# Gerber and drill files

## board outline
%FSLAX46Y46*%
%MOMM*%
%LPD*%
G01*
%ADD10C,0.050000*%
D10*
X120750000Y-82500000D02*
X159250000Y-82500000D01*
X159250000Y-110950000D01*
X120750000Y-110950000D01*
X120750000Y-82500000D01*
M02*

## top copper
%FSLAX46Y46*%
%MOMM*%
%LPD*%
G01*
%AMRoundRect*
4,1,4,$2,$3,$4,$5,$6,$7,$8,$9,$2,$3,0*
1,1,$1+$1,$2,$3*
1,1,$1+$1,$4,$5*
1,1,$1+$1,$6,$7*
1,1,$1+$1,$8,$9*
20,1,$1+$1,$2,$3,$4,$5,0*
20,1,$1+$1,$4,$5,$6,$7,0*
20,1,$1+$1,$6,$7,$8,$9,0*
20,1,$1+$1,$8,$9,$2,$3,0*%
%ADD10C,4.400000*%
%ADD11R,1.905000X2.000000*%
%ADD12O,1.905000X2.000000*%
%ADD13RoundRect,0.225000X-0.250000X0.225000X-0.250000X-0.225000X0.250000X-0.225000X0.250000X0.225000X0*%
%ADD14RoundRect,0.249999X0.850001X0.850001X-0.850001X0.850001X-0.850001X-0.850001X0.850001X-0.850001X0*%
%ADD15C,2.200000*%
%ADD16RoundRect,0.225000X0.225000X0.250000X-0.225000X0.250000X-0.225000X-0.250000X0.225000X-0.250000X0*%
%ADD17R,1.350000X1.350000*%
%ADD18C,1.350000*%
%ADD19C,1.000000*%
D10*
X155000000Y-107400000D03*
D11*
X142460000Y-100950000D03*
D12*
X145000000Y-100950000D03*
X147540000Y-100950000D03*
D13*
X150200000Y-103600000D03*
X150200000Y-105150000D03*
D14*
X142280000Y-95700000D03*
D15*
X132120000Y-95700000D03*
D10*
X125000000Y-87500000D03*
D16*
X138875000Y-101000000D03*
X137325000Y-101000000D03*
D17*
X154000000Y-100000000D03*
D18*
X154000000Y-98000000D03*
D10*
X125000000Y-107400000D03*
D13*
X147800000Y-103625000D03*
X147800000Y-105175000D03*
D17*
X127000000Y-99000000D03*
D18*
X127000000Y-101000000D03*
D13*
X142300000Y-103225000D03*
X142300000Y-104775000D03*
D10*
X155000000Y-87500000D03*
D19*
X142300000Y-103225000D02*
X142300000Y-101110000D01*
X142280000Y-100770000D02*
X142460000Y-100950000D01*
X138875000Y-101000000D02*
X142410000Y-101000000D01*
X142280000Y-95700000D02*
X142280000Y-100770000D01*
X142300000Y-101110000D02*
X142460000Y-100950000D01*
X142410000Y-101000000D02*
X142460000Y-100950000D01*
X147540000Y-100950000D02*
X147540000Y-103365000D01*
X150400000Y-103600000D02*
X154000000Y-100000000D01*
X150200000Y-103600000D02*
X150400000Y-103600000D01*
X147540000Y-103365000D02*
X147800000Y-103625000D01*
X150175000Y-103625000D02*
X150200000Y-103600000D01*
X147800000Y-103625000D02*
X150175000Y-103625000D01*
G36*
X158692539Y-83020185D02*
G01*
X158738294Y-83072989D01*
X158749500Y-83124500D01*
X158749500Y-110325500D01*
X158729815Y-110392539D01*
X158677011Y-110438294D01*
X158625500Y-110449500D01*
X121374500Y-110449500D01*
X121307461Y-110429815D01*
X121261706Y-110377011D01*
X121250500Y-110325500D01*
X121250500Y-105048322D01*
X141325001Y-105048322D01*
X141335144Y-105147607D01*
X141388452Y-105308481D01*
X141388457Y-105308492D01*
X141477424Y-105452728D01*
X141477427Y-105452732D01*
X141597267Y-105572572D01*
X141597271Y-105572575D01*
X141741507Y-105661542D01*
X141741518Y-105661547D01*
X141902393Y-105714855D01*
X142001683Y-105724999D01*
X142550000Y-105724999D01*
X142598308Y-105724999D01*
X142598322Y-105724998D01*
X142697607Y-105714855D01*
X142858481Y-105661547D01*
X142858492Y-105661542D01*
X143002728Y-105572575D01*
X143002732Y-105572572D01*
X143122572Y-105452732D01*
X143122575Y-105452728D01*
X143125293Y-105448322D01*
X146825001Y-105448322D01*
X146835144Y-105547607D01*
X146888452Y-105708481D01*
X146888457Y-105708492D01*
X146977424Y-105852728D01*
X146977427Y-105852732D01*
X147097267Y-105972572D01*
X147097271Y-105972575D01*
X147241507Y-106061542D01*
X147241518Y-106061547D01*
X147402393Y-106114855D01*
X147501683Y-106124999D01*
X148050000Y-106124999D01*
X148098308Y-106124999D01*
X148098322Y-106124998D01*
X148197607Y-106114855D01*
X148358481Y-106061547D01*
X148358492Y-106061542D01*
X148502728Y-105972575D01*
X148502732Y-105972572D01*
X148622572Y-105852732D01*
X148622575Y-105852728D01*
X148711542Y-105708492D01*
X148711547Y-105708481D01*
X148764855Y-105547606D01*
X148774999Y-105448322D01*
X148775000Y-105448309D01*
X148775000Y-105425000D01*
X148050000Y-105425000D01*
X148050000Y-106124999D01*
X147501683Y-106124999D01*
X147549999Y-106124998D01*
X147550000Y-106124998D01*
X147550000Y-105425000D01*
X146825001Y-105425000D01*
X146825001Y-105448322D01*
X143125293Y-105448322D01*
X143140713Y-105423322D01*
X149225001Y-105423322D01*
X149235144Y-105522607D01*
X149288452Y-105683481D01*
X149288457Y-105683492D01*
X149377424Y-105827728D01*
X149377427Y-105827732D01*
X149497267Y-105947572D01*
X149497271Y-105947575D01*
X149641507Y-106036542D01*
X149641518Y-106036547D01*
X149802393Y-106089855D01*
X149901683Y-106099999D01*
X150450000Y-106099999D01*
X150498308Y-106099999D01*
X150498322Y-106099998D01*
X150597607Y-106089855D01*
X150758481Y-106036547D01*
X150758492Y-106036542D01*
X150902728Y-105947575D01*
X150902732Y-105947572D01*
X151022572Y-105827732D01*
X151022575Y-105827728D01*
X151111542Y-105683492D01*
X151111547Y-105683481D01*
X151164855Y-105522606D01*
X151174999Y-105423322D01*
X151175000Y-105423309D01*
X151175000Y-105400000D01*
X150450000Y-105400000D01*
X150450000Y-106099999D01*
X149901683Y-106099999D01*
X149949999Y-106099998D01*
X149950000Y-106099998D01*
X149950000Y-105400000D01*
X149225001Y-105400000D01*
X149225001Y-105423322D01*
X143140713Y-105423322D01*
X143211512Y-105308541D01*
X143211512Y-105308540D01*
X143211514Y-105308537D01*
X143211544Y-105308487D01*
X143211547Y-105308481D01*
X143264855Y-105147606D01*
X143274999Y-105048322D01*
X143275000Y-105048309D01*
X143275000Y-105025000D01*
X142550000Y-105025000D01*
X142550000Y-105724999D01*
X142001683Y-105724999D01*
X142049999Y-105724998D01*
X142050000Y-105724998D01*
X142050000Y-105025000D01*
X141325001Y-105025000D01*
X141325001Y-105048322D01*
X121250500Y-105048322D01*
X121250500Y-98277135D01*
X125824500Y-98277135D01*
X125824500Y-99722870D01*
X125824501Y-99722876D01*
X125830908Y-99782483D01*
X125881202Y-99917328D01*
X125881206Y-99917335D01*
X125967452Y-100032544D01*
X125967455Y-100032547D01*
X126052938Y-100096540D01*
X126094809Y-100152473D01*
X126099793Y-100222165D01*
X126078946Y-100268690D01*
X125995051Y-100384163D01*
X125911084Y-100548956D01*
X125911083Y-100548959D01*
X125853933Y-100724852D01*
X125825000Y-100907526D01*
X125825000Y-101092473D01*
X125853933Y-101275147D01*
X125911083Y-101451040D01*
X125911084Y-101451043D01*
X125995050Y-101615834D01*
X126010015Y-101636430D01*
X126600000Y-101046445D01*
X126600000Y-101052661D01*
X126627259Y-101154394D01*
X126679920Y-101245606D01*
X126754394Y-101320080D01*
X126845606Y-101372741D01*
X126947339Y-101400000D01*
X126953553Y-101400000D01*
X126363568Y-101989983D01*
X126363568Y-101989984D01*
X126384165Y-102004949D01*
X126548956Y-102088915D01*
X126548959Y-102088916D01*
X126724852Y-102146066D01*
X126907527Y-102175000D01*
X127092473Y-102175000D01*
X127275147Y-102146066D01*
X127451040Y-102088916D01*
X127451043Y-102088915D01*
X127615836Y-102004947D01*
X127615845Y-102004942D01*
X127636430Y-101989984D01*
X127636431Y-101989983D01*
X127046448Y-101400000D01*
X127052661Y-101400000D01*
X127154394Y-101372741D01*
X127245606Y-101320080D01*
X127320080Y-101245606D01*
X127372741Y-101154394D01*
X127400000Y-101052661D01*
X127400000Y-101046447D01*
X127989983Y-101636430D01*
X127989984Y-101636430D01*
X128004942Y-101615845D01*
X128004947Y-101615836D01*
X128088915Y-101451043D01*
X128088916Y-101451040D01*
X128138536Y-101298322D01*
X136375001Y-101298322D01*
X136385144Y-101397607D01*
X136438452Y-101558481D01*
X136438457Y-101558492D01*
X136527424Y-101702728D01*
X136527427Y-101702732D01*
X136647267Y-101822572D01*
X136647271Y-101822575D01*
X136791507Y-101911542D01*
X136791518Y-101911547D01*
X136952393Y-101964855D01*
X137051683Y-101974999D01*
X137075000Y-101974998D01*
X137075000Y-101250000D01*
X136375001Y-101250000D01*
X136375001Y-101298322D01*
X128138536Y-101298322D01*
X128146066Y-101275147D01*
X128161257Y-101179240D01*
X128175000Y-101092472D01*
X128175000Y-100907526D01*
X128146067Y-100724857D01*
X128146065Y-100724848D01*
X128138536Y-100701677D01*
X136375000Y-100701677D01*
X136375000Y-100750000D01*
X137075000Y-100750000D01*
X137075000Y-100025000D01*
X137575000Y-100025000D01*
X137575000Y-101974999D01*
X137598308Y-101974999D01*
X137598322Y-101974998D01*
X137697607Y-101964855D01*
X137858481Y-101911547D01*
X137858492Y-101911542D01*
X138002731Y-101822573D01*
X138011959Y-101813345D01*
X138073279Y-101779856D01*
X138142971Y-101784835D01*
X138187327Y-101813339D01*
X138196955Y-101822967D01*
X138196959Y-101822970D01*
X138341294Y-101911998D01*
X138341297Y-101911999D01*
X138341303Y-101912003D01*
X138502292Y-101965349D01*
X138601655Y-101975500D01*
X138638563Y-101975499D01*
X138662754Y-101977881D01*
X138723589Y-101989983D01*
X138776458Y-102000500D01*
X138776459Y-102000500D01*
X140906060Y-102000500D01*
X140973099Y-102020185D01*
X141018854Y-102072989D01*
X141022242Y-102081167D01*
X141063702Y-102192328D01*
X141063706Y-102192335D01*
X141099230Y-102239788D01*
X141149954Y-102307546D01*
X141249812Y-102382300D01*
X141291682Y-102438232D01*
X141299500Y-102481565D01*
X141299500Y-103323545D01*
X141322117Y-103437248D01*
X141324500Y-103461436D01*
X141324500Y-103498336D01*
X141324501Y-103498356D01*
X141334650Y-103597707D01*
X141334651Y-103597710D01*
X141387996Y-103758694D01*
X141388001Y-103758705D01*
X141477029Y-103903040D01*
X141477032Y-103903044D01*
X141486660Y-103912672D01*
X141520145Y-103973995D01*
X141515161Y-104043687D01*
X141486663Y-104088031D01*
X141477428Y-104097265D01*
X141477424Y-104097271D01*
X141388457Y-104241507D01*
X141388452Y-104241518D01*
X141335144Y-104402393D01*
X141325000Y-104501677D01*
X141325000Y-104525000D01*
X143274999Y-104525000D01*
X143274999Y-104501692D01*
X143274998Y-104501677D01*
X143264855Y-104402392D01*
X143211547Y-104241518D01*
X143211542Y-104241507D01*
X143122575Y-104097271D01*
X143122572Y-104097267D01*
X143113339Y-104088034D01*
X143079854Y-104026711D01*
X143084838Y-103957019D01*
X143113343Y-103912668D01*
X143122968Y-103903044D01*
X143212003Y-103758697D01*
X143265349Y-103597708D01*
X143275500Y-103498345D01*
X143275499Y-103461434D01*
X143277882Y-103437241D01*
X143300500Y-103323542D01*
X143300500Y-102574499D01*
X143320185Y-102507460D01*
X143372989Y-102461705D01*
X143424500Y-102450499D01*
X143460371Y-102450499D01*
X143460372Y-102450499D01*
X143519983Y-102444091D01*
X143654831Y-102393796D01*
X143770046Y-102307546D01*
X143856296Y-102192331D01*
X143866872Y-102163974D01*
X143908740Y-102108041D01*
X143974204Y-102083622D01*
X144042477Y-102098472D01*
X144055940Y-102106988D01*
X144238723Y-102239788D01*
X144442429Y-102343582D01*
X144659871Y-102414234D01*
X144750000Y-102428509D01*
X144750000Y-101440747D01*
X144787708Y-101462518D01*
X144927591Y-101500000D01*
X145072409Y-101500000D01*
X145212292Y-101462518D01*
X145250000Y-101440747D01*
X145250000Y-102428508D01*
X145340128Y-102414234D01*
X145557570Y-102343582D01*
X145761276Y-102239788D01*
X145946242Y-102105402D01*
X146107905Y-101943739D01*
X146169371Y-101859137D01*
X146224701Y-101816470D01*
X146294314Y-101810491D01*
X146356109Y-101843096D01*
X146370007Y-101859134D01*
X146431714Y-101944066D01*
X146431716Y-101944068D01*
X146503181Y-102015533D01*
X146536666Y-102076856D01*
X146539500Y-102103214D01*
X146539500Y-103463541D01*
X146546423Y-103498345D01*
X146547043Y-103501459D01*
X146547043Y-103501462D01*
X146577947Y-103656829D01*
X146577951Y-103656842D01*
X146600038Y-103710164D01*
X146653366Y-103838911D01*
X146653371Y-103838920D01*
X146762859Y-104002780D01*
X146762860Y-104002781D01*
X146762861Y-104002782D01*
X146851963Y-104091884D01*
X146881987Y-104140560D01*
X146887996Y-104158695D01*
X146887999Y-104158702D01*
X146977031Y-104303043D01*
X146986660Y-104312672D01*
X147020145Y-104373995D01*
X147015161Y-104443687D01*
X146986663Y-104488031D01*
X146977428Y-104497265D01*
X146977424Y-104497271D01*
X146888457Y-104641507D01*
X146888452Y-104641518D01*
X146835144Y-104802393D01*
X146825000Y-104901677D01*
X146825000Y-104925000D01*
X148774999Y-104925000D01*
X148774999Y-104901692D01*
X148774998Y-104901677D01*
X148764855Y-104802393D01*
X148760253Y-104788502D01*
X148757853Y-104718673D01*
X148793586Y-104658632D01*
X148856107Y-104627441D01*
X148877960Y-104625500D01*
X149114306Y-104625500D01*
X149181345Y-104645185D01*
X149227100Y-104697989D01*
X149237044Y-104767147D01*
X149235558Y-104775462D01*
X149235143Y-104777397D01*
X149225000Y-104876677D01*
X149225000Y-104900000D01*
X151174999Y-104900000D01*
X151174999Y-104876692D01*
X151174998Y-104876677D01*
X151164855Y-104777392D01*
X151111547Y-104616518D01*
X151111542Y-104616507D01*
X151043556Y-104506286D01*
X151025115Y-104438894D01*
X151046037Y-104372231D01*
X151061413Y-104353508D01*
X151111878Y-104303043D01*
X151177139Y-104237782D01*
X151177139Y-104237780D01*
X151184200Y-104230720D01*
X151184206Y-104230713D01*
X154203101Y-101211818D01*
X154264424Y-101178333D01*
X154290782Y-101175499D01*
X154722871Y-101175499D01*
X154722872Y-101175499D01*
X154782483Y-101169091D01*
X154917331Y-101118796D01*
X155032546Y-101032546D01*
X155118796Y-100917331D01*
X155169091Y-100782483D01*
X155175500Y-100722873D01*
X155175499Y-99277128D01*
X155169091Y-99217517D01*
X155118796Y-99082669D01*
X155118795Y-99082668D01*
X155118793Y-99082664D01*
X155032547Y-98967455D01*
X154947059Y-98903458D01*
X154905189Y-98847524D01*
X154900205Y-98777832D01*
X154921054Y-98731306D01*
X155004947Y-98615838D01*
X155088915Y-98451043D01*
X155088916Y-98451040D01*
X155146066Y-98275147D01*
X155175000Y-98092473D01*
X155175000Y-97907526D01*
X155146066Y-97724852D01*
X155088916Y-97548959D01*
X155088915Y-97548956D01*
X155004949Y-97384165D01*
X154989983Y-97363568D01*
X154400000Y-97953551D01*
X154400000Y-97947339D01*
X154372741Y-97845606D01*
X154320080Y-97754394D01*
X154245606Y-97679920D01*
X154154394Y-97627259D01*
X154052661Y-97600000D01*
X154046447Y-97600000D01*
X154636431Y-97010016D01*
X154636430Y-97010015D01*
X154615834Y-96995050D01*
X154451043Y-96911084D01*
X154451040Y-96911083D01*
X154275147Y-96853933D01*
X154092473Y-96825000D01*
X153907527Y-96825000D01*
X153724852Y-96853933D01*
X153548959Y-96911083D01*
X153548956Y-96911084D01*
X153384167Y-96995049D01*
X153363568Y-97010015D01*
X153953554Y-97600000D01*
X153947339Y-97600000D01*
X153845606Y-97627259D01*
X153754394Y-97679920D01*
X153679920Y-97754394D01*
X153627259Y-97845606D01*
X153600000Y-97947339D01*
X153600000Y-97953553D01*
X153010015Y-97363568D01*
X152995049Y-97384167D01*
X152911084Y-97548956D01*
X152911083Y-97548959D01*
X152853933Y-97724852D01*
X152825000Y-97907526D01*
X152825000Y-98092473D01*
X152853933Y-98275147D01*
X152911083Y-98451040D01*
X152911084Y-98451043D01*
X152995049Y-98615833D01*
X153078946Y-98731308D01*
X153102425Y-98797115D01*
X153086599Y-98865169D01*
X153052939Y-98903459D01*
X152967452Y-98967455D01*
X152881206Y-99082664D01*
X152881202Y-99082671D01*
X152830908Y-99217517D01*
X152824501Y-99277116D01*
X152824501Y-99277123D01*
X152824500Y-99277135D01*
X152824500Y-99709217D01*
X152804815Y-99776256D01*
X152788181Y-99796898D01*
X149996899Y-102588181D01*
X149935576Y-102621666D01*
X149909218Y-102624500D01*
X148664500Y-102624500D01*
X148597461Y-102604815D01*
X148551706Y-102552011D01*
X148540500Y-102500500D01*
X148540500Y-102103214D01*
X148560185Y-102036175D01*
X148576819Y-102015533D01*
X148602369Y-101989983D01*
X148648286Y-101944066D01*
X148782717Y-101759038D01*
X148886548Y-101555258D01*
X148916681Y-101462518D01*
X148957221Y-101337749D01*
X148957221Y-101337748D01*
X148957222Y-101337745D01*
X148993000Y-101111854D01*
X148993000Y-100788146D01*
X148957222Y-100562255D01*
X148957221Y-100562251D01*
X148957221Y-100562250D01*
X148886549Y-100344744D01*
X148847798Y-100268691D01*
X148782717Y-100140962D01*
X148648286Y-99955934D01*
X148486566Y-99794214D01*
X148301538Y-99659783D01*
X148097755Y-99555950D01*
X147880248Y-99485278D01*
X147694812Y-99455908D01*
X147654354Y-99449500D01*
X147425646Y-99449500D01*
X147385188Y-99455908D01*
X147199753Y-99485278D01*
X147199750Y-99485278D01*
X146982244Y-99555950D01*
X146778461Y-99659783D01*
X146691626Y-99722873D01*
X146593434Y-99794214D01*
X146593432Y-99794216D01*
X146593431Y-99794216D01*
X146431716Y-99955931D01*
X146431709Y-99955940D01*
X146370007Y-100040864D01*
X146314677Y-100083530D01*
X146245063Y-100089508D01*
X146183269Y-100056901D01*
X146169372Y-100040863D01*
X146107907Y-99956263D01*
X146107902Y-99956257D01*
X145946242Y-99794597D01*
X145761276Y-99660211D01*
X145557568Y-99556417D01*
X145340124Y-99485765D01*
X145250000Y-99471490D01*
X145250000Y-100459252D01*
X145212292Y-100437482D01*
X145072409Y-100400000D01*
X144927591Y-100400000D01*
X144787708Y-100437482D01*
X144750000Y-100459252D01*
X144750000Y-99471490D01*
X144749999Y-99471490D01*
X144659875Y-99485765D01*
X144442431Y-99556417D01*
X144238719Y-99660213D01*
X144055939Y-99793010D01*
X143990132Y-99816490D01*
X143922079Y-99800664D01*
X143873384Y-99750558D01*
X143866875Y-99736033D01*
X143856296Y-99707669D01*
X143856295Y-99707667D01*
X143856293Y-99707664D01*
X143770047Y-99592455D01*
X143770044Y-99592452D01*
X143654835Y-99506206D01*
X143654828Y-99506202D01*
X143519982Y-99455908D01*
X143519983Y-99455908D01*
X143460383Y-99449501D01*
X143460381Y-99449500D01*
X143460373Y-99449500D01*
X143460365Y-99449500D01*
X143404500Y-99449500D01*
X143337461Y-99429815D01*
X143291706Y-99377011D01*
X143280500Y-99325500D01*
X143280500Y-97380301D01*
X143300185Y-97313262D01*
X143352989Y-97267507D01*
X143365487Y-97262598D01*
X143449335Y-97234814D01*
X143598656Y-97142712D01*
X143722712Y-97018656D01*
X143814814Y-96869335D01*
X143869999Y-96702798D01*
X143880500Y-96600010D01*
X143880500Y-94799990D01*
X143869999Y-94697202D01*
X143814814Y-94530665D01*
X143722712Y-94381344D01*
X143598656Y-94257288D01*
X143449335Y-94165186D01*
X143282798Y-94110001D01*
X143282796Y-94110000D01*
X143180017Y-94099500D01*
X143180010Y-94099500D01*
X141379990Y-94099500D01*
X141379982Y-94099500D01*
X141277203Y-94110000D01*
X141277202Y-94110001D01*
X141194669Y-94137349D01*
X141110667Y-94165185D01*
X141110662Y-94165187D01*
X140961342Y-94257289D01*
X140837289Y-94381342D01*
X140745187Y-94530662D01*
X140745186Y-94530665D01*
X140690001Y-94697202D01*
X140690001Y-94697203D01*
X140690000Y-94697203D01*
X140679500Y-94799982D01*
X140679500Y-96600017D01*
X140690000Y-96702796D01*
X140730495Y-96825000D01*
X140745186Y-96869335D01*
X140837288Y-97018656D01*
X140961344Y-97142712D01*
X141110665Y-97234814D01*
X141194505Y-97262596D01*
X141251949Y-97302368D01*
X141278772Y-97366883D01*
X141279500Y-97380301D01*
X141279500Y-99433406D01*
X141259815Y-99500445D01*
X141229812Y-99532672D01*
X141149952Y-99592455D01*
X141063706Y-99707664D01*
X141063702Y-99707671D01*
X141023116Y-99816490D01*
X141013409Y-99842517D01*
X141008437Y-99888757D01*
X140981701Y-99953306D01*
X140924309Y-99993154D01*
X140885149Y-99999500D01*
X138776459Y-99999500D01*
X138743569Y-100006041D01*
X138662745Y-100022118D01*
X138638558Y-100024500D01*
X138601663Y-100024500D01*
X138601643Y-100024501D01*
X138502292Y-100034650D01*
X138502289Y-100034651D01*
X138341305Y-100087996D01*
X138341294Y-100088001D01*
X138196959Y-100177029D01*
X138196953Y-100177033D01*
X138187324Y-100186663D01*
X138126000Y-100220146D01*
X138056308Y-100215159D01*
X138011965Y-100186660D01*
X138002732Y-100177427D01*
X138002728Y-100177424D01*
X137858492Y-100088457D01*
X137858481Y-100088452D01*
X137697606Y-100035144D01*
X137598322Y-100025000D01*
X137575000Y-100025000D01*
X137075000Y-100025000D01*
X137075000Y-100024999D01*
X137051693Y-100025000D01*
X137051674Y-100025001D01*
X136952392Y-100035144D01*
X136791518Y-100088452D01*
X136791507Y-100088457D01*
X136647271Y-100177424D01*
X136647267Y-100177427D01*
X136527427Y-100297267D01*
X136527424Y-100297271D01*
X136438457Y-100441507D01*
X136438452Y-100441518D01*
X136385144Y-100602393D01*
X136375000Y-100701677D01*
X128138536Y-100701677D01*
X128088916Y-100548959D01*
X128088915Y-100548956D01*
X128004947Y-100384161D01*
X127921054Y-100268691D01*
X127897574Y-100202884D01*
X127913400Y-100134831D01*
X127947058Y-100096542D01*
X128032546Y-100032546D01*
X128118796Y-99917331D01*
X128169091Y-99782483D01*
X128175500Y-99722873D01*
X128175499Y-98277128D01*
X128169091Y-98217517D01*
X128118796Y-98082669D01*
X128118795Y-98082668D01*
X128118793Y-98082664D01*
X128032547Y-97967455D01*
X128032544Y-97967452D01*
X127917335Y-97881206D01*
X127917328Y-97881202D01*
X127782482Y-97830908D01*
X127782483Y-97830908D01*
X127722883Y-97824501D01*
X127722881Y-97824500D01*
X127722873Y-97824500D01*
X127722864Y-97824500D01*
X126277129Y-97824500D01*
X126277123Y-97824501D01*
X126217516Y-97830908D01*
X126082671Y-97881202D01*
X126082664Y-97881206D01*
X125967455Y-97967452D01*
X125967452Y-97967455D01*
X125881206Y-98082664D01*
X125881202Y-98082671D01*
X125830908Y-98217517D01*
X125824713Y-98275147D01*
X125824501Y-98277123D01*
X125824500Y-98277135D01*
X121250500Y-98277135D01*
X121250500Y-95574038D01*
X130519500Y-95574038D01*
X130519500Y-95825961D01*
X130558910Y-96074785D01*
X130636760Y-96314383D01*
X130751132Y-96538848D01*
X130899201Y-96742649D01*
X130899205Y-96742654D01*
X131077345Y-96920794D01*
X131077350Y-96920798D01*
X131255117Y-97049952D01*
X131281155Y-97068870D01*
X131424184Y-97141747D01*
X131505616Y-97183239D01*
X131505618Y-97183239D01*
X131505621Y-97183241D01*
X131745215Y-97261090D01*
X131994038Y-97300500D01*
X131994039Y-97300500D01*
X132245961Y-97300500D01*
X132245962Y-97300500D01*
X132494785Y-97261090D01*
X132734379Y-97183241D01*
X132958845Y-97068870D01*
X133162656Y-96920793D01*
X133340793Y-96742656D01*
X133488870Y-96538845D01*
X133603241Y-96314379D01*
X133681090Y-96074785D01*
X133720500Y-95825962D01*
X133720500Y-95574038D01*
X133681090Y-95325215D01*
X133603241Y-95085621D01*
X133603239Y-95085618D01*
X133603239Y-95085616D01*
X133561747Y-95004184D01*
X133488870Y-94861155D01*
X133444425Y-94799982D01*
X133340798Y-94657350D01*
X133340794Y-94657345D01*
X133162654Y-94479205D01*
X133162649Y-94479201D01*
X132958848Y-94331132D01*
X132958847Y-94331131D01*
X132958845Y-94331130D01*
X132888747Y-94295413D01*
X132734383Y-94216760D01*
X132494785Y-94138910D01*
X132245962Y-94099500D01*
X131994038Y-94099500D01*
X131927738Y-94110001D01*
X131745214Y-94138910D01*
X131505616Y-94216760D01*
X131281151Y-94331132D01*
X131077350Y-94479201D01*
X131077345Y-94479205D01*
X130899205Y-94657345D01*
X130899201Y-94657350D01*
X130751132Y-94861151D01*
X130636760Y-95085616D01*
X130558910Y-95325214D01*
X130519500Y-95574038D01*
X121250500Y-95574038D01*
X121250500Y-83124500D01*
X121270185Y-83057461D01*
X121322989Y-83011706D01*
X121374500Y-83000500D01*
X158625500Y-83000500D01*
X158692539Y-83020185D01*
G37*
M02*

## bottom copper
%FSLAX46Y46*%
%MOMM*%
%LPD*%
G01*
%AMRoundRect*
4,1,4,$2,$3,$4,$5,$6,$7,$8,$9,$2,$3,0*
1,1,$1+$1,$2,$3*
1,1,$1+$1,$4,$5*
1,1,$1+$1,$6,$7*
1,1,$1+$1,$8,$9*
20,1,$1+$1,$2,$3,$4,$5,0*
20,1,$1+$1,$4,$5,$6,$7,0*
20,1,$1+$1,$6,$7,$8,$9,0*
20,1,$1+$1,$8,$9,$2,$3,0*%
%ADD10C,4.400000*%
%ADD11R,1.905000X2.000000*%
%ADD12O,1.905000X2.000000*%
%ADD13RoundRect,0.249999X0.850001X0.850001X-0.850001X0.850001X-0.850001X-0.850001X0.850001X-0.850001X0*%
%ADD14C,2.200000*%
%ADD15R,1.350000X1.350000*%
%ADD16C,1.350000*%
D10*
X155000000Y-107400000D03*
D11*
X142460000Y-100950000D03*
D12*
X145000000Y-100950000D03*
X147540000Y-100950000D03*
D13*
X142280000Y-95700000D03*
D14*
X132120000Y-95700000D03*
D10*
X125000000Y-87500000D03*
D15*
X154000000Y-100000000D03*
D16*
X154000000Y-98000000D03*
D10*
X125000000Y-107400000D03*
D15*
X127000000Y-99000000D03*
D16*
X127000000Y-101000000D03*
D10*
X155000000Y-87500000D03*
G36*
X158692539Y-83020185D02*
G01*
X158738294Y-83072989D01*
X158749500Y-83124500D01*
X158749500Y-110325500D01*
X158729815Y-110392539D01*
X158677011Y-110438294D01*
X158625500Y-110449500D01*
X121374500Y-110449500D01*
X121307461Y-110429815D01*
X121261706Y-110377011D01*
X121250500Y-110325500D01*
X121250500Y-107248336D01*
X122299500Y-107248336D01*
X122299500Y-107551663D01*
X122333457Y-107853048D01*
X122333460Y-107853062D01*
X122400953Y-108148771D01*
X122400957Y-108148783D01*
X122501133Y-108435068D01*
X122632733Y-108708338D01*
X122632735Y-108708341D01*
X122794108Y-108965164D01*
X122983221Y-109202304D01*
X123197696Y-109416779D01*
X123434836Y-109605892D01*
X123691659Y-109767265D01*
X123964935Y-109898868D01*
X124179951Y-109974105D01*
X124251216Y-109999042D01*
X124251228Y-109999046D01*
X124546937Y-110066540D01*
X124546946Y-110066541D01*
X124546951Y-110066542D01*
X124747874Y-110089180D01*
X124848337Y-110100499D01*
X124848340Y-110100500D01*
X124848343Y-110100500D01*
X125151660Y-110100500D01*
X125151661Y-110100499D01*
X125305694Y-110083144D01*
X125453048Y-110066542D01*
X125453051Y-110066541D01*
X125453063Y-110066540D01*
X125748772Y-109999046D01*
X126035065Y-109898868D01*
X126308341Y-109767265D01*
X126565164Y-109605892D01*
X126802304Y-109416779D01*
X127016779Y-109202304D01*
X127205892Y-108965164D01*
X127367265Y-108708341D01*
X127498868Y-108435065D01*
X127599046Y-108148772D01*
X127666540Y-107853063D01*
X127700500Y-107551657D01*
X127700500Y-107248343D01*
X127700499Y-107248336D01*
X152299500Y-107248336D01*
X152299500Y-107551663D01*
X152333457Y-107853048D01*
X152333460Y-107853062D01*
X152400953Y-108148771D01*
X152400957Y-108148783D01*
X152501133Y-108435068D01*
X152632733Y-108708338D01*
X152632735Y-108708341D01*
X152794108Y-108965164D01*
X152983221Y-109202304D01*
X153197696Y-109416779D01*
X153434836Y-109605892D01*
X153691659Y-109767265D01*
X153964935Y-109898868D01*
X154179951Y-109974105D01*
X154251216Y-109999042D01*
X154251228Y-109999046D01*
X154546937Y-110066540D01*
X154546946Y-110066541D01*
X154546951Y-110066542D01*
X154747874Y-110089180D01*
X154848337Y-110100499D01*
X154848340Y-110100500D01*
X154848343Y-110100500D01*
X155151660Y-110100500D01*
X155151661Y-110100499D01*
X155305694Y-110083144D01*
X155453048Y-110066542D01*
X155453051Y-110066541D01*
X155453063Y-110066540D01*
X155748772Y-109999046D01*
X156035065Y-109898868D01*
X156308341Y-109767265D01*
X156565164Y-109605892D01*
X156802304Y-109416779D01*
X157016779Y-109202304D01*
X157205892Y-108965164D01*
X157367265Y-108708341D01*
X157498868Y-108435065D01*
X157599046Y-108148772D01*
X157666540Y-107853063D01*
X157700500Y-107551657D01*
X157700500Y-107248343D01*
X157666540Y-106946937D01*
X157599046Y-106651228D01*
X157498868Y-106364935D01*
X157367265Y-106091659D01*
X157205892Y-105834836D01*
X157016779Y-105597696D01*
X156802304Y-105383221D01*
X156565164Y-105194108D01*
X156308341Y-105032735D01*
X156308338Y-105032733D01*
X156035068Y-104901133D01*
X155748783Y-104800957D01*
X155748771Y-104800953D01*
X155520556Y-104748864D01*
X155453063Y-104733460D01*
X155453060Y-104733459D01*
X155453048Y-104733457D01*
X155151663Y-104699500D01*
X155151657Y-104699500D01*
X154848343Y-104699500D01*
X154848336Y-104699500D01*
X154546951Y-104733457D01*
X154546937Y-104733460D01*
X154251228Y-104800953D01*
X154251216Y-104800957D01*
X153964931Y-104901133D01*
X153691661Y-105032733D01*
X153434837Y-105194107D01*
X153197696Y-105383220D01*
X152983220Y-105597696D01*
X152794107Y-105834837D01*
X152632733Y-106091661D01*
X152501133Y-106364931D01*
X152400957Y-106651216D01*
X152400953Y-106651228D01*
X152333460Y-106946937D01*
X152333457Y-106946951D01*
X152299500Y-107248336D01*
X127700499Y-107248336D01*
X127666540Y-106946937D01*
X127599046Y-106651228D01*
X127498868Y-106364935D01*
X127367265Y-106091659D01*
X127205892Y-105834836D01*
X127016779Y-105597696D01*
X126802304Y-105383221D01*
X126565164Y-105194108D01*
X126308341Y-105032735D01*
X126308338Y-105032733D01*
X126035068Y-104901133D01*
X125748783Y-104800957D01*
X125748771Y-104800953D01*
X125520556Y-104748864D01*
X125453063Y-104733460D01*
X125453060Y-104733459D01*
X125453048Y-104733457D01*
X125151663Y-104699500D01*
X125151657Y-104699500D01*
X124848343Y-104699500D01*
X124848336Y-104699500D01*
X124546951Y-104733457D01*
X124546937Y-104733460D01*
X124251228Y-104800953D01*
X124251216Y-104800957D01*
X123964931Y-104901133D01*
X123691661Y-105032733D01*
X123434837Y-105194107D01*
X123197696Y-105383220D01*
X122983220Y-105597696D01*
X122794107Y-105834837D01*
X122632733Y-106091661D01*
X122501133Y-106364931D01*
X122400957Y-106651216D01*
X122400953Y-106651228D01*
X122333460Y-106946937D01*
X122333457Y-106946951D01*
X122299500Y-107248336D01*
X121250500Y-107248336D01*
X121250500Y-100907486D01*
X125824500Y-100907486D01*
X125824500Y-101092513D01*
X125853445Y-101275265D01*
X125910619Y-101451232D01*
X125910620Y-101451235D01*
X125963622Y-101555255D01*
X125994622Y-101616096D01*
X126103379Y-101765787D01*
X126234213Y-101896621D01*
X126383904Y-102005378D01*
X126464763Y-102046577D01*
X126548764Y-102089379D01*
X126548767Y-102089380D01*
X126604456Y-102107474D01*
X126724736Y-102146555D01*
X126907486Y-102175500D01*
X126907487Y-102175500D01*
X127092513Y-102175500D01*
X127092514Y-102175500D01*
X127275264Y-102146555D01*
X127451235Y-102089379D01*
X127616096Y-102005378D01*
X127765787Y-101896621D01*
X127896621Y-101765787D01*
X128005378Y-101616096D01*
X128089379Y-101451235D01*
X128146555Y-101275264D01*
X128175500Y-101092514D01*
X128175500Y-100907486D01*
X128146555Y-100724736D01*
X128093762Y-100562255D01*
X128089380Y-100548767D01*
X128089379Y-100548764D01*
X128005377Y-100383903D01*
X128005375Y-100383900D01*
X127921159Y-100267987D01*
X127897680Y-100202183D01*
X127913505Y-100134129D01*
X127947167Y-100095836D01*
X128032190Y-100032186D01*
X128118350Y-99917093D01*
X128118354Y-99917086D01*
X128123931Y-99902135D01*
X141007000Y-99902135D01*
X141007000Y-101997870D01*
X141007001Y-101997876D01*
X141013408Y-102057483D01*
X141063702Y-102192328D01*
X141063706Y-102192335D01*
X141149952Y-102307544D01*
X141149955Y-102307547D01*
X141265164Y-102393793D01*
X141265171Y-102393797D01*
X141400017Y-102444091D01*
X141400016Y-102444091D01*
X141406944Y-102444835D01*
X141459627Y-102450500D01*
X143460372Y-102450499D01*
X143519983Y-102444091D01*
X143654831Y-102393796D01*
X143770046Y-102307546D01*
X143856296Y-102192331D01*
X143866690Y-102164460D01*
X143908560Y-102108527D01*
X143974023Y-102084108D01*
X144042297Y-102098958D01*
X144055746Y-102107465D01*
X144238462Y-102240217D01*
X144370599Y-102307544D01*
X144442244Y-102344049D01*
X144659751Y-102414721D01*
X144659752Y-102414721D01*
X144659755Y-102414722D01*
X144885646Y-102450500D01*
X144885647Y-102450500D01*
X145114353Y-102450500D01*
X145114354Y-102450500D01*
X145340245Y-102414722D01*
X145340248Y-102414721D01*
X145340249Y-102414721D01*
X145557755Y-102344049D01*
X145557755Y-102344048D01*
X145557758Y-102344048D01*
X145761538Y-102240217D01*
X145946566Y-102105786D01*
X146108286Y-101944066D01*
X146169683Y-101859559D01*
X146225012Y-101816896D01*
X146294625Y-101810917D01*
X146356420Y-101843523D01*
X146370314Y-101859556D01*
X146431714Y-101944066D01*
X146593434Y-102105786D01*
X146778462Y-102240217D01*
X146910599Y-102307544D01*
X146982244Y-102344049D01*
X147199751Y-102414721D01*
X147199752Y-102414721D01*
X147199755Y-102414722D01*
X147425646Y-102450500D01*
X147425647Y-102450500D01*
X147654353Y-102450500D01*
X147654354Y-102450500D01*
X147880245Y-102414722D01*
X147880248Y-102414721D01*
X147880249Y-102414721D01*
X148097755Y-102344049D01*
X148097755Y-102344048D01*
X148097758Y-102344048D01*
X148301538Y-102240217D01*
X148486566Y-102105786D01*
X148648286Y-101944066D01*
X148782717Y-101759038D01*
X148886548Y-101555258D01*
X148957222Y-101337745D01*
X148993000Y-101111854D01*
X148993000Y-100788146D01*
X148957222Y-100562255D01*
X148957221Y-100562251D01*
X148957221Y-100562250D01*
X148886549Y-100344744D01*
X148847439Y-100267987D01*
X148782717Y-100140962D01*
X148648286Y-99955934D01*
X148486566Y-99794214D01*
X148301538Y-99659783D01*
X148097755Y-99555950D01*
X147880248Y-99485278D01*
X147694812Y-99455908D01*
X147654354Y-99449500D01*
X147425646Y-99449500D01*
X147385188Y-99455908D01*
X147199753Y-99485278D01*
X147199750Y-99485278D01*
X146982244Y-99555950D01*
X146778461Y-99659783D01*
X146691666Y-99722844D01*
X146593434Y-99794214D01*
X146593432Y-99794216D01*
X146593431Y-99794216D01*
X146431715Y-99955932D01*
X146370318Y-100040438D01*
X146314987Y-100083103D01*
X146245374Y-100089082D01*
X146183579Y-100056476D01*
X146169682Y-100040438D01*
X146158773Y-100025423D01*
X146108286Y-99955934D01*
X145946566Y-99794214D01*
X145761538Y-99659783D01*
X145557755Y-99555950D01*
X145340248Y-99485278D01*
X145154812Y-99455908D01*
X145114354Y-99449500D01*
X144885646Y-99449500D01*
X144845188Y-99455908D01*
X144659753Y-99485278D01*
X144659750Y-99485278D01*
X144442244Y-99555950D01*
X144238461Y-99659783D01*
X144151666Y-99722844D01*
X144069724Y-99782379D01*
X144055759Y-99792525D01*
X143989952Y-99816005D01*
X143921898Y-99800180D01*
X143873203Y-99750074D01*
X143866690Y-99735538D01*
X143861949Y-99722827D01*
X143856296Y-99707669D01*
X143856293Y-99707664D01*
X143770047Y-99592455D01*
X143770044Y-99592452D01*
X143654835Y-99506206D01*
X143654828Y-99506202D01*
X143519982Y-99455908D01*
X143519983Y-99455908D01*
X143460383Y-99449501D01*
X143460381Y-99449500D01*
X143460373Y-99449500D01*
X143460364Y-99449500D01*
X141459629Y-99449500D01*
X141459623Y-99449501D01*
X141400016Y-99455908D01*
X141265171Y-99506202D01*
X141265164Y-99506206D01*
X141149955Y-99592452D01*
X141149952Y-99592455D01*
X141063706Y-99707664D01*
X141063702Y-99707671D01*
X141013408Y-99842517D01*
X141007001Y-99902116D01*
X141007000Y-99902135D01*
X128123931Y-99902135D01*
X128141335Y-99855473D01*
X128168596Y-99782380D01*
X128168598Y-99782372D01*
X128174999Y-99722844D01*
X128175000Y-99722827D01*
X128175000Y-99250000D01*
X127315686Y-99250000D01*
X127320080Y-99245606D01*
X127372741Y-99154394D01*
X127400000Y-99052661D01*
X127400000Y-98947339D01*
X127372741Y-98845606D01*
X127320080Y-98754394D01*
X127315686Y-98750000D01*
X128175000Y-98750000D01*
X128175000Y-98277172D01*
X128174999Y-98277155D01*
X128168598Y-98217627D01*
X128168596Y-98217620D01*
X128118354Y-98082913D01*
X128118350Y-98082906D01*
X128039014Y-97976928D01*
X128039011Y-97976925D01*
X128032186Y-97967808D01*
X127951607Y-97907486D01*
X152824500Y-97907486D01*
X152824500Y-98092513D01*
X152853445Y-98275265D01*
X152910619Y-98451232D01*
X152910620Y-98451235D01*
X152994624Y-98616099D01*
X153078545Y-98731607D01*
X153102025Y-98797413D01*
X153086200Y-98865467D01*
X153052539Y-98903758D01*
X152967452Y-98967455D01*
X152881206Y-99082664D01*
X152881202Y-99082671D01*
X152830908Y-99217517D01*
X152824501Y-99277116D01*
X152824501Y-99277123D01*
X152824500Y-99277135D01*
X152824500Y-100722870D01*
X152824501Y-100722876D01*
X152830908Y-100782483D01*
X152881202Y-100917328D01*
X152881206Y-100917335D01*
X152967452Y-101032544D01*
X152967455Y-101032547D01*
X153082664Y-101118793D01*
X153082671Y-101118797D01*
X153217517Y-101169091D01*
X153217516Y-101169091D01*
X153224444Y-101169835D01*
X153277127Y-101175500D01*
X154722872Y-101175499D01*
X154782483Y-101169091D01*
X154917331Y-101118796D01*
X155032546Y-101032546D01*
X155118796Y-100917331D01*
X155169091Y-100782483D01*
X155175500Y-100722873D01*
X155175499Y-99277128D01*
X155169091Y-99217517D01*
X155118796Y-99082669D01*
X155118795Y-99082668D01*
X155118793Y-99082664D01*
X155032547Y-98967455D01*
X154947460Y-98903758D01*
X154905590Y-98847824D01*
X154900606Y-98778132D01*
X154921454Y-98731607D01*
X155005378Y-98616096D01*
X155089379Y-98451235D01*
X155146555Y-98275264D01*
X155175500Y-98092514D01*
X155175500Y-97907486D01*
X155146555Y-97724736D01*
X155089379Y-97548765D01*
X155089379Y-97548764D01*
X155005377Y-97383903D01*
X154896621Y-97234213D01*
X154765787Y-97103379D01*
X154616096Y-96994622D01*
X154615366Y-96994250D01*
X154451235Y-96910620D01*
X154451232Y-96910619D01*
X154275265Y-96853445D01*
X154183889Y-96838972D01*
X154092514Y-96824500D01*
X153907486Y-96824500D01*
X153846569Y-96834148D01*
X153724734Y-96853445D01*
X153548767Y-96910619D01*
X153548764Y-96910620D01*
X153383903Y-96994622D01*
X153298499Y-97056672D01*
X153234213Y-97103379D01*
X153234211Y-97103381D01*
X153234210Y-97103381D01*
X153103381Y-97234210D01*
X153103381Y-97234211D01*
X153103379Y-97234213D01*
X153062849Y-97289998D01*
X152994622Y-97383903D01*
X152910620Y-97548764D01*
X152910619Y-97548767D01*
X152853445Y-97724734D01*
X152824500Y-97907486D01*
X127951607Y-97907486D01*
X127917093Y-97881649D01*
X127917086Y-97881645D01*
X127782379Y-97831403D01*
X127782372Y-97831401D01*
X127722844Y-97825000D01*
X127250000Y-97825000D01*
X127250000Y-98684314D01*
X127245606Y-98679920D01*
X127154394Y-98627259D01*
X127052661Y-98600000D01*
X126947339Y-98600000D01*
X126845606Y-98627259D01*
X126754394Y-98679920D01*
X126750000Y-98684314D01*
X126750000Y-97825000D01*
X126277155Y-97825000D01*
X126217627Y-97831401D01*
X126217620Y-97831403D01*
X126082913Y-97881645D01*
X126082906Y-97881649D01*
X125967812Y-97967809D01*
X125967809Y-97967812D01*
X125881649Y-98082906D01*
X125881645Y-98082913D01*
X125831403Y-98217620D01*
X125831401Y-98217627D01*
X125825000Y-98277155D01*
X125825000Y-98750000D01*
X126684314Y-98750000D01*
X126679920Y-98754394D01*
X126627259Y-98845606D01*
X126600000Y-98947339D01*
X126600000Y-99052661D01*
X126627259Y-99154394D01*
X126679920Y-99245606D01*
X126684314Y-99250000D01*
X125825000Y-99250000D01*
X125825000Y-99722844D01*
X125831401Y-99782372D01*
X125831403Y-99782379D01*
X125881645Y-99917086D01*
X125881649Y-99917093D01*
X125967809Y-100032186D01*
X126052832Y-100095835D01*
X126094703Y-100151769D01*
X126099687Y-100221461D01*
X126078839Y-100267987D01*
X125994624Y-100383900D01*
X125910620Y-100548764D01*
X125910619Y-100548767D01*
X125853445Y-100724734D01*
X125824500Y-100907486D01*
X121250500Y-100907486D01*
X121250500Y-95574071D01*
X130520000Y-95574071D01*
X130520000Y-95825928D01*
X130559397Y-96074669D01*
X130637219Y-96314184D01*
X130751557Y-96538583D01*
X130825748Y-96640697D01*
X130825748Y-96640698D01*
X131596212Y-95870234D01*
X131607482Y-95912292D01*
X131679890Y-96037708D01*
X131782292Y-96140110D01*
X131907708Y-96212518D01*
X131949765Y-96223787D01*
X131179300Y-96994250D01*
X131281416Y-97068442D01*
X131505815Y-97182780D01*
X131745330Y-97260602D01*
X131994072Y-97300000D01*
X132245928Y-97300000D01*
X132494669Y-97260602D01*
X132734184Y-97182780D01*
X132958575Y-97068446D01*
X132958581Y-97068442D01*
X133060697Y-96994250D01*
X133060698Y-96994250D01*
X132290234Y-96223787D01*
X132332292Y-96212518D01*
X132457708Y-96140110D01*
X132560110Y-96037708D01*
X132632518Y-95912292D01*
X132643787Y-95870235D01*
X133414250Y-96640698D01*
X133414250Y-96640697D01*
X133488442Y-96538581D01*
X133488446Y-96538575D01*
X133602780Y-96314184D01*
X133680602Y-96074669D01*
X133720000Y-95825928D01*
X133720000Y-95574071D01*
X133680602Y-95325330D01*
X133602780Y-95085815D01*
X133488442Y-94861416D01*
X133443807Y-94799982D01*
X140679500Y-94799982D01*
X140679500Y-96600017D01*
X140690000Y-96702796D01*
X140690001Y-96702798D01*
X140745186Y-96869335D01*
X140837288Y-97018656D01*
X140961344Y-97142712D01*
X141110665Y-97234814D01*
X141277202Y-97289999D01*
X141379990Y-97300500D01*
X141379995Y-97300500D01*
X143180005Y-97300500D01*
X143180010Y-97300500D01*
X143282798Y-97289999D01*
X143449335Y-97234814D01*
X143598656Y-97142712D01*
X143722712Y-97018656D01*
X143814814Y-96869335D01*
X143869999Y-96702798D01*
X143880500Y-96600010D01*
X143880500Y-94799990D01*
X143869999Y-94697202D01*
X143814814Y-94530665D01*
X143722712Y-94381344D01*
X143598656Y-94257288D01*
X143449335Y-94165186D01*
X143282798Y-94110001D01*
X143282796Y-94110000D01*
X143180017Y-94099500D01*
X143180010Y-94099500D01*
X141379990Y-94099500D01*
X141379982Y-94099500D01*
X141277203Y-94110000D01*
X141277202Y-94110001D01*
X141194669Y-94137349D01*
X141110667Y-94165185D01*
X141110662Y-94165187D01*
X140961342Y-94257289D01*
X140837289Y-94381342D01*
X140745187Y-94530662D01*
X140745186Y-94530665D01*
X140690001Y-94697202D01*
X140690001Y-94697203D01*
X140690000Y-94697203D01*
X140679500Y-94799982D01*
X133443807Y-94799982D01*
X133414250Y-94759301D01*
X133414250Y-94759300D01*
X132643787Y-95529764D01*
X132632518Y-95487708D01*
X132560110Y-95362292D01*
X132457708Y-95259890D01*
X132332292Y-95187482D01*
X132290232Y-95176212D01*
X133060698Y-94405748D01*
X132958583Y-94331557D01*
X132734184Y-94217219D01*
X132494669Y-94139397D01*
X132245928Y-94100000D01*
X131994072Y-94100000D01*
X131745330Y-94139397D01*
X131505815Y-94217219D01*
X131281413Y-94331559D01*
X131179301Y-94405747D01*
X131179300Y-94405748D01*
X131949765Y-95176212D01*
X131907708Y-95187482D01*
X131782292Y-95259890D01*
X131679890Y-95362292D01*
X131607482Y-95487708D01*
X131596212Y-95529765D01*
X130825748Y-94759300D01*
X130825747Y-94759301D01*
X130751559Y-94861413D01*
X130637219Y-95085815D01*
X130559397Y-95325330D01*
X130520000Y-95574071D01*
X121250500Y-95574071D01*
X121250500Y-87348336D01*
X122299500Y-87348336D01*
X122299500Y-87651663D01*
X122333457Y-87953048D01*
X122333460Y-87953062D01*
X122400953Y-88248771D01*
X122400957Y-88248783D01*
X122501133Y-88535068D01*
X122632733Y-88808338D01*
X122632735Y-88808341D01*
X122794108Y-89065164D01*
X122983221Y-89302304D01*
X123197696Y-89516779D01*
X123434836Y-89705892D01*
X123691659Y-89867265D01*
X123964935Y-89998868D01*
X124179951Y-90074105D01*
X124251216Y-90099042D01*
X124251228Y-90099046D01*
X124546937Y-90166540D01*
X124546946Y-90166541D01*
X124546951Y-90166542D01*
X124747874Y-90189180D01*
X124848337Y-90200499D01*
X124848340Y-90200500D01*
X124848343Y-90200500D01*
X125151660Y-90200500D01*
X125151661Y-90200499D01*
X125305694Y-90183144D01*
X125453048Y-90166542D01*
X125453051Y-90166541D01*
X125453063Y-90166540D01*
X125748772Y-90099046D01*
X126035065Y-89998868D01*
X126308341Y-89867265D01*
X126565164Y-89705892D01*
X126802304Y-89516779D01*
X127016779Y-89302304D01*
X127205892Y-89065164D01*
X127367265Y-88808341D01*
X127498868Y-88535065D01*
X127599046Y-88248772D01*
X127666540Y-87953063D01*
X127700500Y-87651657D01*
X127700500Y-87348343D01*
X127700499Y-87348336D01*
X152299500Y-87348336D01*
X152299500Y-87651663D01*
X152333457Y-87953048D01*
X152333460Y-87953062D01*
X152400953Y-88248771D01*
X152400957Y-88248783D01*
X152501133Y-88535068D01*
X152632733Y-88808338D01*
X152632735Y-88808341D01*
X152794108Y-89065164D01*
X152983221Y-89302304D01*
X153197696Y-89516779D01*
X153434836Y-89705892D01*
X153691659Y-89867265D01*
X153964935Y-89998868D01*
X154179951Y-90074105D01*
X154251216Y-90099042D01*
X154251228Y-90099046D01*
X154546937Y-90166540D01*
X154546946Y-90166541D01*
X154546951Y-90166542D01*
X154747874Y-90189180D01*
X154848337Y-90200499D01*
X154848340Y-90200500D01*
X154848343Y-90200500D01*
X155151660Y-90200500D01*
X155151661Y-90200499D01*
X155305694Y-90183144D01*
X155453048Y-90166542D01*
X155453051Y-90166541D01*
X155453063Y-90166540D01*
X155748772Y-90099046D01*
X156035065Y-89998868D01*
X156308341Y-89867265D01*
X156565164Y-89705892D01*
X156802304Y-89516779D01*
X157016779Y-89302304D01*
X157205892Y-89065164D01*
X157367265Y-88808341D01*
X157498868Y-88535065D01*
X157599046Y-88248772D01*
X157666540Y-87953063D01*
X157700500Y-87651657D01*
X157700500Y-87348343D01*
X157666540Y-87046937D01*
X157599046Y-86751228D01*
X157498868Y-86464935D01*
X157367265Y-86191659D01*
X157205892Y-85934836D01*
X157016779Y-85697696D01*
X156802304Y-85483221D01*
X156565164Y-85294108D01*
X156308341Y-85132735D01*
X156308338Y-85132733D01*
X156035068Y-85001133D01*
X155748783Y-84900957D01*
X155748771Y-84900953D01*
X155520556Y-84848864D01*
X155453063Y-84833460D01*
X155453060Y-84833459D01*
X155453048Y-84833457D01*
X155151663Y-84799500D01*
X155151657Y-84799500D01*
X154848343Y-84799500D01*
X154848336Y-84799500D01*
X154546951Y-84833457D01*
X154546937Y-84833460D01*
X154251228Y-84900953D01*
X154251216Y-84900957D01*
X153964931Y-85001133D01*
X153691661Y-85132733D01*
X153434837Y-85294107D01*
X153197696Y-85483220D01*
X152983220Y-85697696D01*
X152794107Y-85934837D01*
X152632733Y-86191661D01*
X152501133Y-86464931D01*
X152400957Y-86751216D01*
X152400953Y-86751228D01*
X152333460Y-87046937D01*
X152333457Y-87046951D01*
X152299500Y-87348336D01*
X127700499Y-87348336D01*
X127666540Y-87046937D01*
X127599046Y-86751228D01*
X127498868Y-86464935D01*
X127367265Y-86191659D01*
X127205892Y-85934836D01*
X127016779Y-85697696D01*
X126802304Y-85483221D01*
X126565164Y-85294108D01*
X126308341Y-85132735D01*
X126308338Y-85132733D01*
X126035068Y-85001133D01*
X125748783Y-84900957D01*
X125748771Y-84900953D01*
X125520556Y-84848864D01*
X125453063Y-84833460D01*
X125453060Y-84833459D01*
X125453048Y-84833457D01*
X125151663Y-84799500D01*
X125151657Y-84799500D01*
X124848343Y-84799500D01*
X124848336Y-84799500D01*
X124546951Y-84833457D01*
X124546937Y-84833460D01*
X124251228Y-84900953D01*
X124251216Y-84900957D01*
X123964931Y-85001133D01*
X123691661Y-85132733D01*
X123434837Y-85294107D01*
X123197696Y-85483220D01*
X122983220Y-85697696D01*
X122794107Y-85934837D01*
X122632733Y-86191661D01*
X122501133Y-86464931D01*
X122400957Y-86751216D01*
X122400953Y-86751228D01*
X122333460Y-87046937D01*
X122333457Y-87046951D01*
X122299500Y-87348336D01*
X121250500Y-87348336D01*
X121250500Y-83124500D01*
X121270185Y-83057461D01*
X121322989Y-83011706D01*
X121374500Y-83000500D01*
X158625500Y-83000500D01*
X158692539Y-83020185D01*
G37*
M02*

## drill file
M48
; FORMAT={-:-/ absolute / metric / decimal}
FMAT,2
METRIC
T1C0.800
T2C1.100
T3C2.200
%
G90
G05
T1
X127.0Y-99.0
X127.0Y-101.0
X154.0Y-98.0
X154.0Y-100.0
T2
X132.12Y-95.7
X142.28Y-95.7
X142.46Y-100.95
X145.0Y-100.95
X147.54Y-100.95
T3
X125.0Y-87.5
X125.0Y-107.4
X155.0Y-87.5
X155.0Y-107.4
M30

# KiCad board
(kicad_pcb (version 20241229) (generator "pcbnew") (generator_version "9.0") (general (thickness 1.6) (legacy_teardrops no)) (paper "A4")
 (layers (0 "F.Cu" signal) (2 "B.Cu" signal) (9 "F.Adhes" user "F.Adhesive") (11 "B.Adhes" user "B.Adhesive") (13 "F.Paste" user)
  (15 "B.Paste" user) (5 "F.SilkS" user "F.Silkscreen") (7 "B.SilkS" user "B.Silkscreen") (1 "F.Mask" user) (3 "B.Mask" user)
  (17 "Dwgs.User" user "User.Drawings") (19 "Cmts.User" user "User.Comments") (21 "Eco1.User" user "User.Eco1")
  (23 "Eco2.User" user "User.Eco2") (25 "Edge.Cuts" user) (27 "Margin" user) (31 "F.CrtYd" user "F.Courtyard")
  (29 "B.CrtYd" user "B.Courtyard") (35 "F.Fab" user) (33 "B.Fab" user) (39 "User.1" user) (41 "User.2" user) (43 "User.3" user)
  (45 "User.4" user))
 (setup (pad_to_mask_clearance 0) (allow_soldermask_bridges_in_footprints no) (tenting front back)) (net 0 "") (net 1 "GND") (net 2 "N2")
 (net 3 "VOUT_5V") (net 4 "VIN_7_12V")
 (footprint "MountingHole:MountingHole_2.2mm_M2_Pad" (layer "F.Cu") (at 155 107.4)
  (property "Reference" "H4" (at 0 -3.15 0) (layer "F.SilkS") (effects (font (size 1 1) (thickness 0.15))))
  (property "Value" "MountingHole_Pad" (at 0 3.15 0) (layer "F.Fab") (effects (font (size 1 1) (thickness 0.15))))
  (pad "1" thru_hole circle (at 0 0) (size 4.4 4.4) (drill 2.2) (layers "*.Cu" "*.Mask") (remove_unused_layers no) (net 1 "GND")
   (zone_connect 2)))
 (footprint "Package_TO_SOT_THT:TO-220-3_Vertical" (layer "F.Cu") (at 142.46 100.95)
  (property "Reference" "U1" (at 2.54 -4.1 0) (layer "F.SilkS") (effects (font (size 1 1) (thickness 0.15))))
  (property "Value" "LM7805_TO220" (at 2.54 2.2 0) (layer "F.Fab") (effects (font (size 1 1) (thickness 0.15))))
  (pad "1" thru_hole rect (at 0 0) (size 1.905 2) (drill 1.1) (layers "*.Cu" "*.Mask") (remove_unused_layers no) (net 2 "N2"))
  (pad "2" thru_hole oval (at 2.54 0) (size 1.905 2) (drill 1.1) (layers "*.Cu" "*.Mask") (remove_unused_layers no) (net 1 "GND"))
  (pad "3" thru_hole oval (at 5.08 0) (size 1.905 2) (drill 1.1) (layers "*.Cu" "*.Mask") (remove_unused_layers no) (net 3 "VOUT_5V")))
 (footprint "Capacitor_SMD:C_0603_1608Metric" (layer "F.Cu") (at 150.2 104.375 -90)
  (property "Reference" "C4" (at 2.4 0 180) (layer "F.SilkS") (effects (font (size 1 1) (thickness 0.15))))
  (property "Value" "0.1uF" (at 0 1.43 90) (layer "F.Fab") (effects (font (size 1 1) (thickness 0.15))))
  (pad "1" smd roundrect (at -0.775 0 270) (size 0.9 0.95) (layers "F.Cu" "F.Mask" "F.Paste") (roundrect_rratio 0.25) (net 3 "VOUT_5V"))
  (pad "2" smd roundrect (at 0.775 0 270) (size 0.9 0.95) (layers "F.Cu" "F.Mask" "F.Paste") (roundrect_rratio 0.25) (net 1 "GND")))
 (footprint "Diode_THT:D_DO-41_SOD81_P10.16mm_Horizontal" (layer "F.Cu") (at 142.28 95.7 180)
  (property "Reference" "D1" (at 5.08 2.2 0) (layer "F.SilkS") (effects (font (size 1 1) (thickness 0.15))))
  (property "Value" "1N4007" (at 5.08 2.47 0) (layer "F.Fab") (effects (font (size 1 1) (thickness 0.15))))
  (pad "1" thru_hole roundrect (at 0 0 180) (size 2.2 2.2) (drill 1.1) (layers "*.Cu" "*.Mask") (remove_unused_layers no)
   (roundrect_rratio 0.113636) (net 2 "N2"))
  (pad "2" thru_hole circle (at 10.16 0 180) (size 2.2 2.2) (drill 1.1) (layers "*.Cu" "*.Mask") (remove_unused_layers no)
   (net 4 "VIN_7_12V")))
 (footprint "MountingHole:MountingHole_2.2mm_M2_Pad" (layer "F.Cu") (at 125 87.5)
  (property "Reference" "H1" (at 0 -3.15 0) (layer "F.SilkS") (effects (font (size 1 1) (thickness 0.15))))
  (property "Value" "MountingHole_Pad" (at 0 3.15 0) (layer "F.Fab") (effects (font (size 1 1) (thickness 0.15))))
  (pad "1" thru_hole circle (at 0 0) (size 4.4 4.4) (drill 2.2) (layers "*.Cu" "*.Mask") (remove_unused_layers no) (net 1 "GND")
   (zone_connect 2)))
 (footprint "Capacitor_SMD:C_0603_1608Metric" (layer "F.Cu") (at 138.1 101 180)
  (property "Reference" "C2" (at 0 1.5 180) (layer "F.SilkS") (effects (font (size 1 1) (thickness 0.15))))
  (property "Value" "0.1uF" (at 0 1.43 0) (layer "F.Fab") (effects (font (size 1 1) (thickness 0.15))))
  (pad "1" smd roundrect (at -0.775 0 180) (size 0.9 0.95) (layers "F.Cu" "F.Mask" "F.Paste") (roundrect_rratio 0.25) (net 2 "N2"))
  (pad "2" smd roundrect (at 0.775 0 180) (size 0.9 0.95) (layers "F.Cu" "F.Mask" "F.Paste") (roundrect_rratio 0.25) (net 1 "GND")))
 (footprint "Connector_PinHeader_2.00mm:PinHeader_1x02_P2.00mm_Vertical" (layer "F.Cu") (at 154 100 180)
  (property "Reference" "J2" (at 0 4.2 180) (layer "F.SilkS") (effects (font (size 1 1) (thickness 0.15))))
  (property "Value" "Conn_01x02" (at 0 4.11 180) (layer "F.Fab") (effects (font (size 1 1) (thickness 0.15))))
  (pad "1" thru_hole rect (at 0 0 180) (size 1.35 1.35) (drill 0.8) (layers "*.Cu" "*.Mask") (remove_unused_layers no) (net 3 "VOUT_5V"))
  (pad "2" thru_hole circle (at 0 2 180) (size 1.35 1.35) (drill 0.8) (layers "*.Cu" "*.Mask") (remove_unused_layers no) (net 1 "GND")))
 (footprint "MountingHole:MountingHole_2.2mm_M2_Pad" (layer "F.Cu") (at 125 107.4)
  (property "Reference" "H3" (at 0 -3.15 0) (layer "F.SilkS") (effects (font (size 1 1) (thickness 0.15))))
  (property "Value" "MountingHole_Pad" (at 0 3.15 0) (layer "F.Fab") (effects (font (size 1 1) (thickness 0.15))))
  (pad "1" thru_hole circle (at 0 0) (size 4.4 4.4) (drill 2.2) (layers "*.Cu" "*.Mask") (remove_unused_layers no) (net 1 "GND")
   (zone_connect 2)))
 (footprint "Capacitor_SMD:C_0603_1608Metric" (layer "F.Cu") (at 147.8 104.4 -90)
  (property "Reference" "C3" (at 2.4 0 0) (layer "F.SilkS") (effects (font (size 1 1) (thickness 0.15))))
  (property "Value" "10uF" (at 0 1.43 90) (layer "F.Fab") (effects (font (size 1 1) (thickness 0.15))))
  (pad "1" smd roundrect (at -0.775 0 270) (size 0.9 0.95) (layers "F.Cu" "F.Mask" "F.Paste") (roundrect_rratio 0.25) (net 3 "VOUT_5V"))
  (pad "2" smd roundrect (at 0.775 0 270) (size 0.9 0.95) (layers "F.Cu" "F.Mask" "F.Paste") (roundrect_rratio 0.25) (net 1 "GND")))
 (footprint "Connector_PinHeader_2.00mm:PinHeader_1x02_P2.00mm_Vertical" (layer "F.Cu") (at 127 99)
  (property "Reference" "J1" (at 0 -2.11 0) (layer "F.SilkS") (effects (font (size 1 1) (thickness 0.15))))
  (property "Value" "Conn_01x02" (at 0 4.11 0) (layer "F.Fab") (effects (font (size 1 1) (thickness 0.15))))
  (pad "1" thru_hole rect (at 0 0) (size 1.35 1.35) (drill 0.8) (layers "*.Cu" "*.Mask") (remove_unused_layers no) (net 4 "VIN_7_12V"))
  (pad "2" thru_hole circle (at 0 2) (size 1.35 1.35) (drill 0.8) (layers "*.Cu" "*.Mask") (remove_unused_layers no) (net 1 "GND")))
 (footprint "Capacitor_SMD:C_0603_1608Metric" (layer "F.Cu") (at 142.3 104 -90)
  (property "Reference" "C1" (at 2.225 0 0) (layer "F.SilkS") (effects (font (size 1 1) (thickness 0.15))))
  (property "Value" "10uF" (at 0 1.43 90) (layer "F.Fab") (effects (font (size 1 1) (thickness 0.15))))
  (pad "1" smd roundrect (at -0.775 0 270) (size 0.9 0.95) (layers "F.Cu" "F.Mask" "F.Paste") (roundrect_rratio 0.25) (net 2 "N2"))
  (pad "2" smd roundrect (at 0.775 0 270) (size 0.9 0.95) (layers "F.Cu" "F.Mask" "F.Paste") (roundrect_rratio 0.25) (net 1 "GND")))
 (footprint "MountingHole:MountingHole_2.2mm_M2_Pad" (layer "F.Cu") (at 155 87.5)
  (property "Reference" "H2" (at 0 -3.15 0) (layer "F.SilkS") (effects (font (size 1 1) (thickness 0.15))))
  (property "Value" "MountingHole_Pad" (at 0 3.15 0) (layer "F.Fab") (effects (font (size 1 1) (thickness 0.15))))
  (pad "1" thru_hole circle (at 0 0) (size 4.4 4.4) (drill 2.2) (layers "*.Cu" "*.Mask") (remove_unused_layers no) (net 1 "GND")
   (zone_connect 2)))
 (gr_rect (start 120.75 82.5) (end 159.25 110.95) (stroke (width 0.05) (type default)) (fill no) (layer "Edge.Cuts"))
 (segment (start 142.3 103.225) (end 142.3 101.11) (width 1) (layer "F.Cu") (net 2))
 (segment (start 142.28 100.77) (end 142.46 100.95) (width 1) (layer "F.Cu") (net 2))
 (segment (start 138.875 101) (end 142.41 101) (width 1) (layer "F.Cu") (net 2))
 (segment (start 142.28 95.7) (end 142.28 100.77) (width 1) (layer "F.Cu") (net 2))
 (segment (start 142.3 101.11) (end 142.46 100.95) (width 1) (layer "F.Cu") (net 2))
 (segment (start 142.41 101) (end 142.46 100.95) (width 1) (layer "F.Cu") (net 2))
 (segment (start 147.54 100.95) (end 147.54 103.365) (width 1) (layer "F.Cu") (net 3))
 (segment (start 150.4 103.6) (end 154 100) (width 1) (layer "F.Cu") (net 3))
 (segment (start 150.2 103.6) (end 150.4 103.6) (width 1) (layer "F.Cu") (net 3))
 (segment (start 147.54 103.365) (end 147.8 103.625) (width 1) (layer "F.Cu") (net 3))
 (segment (start 150.175 103.625) (end 150.2 103.6) (width 1) (layer "F.Cu") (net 3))
 (segment (start 147.8 103.625) (end 150.175 103.625) (width 1) (layer "F.Cu") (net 3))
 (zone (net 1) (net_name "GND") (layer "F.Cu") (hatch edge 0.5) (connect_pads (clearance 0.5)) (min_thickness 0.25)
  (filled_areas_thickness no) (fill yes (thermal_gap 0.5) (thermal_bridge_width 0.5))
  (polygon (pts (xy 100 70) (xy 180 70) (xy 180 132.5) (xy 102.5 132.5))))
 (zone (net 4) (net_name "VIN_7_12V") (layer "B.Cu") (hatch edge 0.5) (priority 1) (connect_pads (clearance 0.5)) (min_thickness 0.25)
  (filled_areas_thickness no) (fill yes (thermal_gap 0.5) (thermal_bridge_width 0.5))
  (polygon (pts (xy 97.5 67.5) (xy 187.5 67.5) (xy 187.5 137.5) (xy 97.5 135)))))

